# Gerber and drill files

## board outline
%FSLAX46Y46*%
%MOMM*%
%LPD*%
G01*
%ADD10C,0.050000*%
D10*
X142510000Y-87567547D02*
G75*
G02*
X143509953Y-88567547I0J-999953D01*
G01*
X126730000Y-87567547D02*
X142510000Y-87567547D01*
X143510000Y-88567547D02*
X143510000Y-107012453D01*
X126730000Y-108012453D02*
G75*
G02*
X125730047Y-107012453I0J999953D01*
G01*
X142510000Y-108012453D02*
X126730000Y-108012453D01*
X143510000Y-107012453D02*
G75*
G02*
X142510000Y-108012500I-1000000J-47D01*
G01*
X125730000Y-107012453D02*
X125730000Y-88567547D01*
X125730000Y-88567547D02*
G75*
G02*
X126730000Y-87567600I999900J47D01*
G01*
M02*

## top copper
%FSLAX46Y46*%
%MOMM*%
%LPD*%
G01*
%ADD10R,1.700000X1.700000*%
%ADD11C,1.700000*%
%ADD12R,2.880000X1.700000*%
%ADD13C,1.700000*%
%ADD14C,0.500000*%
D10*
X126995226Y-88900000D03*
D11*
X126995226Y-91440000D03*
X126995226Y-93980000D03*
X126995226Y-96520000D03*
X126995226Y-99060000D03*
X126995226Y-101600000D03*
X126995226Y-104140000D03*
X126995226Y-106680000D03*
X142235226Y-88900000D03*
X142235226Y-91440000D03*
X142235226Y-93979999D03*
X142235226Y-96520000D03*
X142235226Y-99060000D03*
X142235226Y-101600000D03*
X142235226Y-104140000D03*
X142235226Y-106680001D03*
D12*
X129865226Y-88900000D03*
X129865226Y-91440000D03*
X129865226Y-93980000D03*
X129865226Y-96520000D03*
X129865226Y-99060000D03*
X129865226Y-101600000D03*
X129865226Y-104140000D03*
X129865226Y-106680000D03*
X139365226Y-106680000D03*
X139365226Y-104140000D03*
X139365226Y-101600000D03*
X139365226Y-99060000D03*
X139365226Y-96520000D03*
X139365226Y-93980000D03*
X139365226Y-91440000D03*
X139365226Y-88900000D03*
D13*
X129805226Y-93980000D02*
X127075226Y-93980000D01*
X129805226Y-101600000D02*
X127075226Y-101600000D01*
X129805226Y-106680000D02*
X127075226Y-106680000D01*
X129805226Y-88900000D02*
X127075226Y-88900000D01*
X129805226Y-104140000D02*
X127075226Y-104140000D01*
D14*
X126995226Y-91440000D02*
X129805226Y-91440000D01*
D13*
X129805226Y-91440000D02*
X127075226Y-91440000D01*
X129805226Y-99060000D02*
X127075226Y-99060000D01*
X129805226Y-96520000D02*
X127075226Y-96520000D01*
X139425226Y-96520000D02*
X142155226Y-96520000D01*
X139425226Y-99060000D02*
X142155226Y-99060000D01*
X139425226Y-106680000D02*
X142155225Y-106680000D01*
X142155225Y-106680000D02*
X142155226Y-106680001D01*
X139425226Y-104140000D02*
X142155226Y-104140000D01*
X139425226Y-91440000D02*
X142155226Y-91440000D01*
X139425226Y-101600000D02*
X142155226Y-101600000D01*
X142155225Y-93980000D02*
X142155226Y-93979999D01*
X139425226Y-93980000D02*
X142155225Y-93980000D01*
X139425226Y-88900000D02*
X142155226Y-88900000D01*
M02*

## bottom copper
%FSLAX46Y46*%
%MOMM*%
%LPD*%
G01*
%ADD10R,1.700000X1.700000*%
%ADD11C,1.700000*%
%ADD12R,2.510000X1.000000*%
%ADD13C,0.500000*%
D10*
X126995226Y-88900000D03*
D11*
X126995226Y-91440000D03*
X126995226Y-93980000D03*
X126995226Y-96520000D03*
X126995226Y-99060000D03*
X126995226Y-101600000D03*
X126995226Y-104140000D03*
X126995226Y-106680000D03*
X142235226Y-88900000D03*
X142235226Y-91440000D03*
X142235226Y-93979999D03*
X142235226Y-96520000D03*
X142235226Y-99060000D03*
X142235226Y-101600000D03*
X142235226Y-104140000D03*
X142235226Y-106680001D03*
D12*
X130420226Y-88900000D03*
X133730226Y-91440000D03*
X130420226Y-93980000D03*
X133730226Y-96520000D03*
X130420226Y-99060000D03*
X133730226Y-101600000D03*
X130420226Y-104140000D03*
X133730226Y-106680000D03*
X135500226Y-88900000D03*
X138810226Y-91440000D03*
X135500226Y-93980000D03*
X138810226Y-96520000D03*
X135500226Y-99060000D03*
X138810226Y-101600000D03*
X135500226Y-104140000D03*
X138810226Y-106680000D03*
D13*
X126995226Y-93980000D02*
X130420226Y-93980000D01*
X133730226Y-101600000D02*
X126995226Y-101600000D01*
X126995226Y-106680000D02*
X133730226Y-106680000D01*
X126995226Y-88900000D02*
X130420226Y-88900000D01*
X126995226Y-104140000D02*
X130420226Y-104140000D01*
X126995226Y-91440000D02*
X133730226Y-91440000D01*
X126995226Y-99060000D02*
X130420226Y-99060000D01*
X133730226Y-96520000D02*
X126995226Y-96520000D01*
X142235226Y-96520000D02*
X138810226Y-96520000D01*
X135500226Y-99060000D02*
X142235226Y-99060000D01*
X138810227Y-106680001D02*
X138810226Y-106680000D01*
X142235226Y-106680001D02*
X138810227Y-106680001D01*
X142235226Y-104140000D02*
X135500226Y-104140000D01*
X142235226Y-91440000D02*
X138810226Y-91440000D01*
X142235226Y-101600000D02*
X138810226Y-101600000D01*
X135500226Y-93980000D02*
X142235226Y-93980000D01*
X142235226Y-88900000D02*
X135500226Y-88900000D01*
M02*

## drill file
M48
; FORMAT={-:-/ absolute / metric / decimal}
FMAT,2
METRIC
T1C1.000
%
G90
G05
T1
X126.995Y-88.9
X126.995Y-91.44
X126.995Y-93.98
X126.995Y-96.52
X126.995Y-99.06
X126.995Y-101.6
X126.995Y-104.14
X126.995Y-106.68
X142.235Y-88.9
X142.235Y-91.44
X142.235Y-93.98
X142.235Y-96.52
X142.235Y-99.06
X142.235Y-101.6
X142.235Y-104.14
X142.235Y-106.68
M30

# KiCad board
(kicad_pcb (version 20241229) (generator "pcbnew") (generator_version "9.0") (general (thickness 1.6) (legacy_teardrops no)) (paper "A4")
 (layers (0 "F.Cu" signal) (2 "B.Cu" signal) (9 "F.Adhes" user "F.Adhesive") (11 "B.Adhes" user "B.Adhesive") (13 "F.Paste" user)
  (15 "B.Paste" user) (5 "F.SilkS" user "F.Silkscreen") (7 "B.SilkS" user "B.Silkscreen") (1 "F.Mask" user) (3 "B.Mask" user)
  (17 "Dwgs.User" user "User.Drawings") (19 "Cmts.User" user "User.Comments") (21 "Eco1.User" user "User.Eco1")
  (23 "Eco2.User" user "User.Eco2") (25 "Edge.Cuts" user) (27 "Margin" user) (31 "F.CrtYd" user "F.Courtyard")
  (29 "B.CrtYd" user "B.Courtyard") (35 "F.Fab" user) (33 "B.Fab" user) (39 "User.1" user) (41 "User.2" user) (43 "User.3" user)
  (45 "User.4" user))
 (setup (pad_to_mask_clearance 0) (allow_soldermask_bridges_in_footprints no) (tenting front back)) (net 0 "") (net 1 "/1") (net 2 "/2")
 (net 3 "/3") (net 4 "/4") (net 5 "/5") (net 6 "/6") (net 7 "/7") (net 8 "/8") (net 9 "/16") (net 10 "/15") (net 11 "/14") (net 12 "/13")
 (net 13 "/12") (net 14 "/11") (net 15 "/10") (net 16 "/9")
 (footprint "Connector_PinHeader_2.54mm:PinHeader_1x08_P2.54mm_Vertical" (layer "F.Cu") (at 126.995226 88.9)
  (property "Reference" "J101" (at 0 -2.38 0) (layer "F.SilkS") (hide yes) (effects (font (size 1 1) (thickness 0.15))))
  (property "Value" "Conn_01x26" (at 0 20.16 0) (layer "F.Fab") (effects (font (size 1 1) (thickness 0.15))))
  (pad "1" thru_hole rect (at 0 0) (size 1.7 1.7) (drill 1) (layers "*.Cu" "*.Mask") (remove_unused_layers no) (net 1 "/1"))
  (pad "2" thru_hole circle (at 0 2.54) (size 1.7 1.7) (drill 1) (layers "*.Cu" "*.Mask") (remove_unused_layers no) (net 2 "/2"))
  (pad "3" thru_hole circle (at 0 5.08) (size 1.7 1.7) (drill 1) (layers "*.Cu" "*.Mask") (remove_unused_layers no) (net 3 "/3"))
  (pad "4" thru_hole circle (at 0 7.62) (size 1.7 1.7) (drill 1) (layers "*.Cu" "*.Mask") (remove_unused_layers no) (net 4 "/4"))
  (pad "5" thru_hole circle (at 0 10.16) (size 1.7 1.7) (drill 1) (layers "*.Cu" "*.Mask") (remove_unused_layers no) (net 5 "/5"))
  (pad "6" thru_hole circle (at 0 12.7) (size 1.7 1.7) (drill 1) (layers "*.Cu" "*.Mask") (remove_unused_layers no) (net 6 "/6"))
  (pad "7" thru_hole circle (at 0 15.24) (size 1.7 1.7) (drill 1) (layers "*.Cu" "*.Mask") (remove_unused_layers no) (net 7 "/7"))
  (pad "8" thru_hole circle (at 0 17.78) (size 1.7 1.7) (drill 1) (layers "*.Cu" "*.Mask") (remove_unused_layers no) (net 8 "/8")))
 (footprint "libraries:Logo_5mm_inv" (layer "F.Cu") (at 134.617351 90.17)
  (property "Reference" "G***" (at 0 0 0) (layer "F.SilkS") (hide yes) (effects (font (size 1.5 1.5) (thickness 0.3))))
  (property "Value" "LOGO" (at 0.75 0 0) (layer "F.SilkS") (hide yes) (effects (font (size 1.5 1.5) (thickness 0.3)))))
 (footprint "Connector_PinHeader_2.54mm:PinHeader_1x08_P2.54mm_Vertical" (layer "F.Cu") (at 142.235226 88.9)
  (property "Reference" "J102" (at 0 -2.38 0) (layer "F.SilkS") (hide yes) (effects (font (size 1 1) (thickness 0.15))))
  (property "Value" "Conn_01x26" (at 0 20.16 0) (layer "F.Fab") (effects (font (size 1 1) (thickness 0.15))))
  (pad "1" thru_hole circle (at 0 0) (size 1.7 1.7) (drill 1) (layers "*.Cu" "*.Mask") (remove_unused_layers no) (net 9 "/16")
   (thermal_bridge_angle 90))
  (pad "2" thru_hole circle (at 0 2.54) (size 1.7 1.7) (drill 1) (layers "*.Cu" "*.Mask") (remove_unused_layers no) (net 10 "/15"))
  (pad "3" thru_hole circle (at 0 5.079999) (size 1.7 1.7) (drill 1) (layers "*.Cu" "*.Mask") (remove_unused_layers no) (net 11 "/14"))
  (pad "4" thru_hole circle (at 0 7.62) (size 1.7 1.7) (drill 1) (layers "*.Cu" "*.Mask") (remove_unused_layers no) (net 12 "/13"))
  (pad "5" thru_hole circle (at 0 10.16) (size 1.7 1.7) (drill 1) (layers "*.Cu" "*.Mask") (remove_unused_layers no) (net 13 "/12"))
  (pad "6" thru_hole circle (at 0 12.7) (size 1.7 1.7) (drill 1) (layers "*.Cu" "*.Mask") (remove_unused_layers no) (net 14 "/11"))
  (pad "7" thru_hole circle (at 0 15.24) (size 1.7 1.7) (drill 1) (layers "*.Cu" "*.Mask") (remove_unused_layers no) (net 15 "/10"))
  (pad "8" thru_hole circle (at 0 17.780001) (size 1.7 1.7) (drill 1) (layers "*.Cu" "*.Mask") (remove_unused_layers no) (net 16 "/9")))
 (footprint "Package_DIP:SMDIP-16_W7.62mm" (layer "F.Cu") (at 134.615226 97.79)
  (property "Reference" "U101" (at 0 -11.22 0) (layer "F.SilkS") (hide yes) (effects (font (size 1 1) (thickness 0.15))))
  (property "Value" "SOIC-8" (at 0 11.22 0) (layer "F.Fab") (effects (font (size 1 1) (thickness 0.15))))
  (pad "1" smd rect (at -4.75 -8.89) (size 2.88 1.7) (layers "F.Cu" "F.Mask" "F.Paste") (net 1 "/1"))
  (pad "2" smd rect (at -4.75 -6.35) (size 2.88 1.7) (layers "F.Cu" "F.Mask" "F.Paste") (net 2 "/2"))
  (pad "3" smd rect (at -4.75 -3.81) (size 2.88 1.7) (layers "F.Cu" "F.Mask" "F.Paste") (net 3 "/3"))
  (pad "4" smd rect (at -4.75 -1.27) (size 2.88 1.7) (layers "F.Cu" "F.Mask" "F.Paste") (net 4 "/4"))
  (pad "5" smd rect (at -4.75 1.27) (size 2.88 1.7) (layers "F.Cu" "F.Mask" "F.Paste") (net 5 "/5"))
  (pad "6" smd rect (at -4.75 3.81) (size 2.88 1.7) (layers "F.Cu" "F.Mask" "F.Paste") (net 6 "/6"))
  (pad "7" smd rect (at -4.75 6.35) (size 2.88 1.7) (layers "F.Cu" "F.Mask" "F.Paste") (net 7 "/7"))
  (pad "8" smd rect (at -4.75 8.89) (size 2.88 1.7) (layers "F.Cu" "F.Mask" "F.Paste") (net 8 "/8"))
  (pad "9" smd rect (at 4.75 8.89) (size 2.88 1.7) (layers "F.Cu" "F.Mask" "F.Paste") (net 16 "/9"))
  (pad "10" smd rect (at 4.75 6.35) (size 2.88 1.7) (layers "F.Cu" "F.Mask" "F.Paste") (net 15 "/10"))
  (pad "11" smd rect (at 4.75 3.81) (size 2.88 1.7) (layers "F.Cu" "F.Mask" "F.Paste") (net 14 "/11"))
  (pad "12" smd rect (at 4.75 1.27) (size 2.88 1.7) (layers "F.Cu" "F.Mask" "F.Paste") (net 13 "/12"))
  (pad "13" smd rect (at 4.75 -1.27) (size 2.88 1.7) (layers "F.Cu" "F.Mask" "F.Paste") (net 12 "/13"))
  (pad "14" smd rect (at 4.75 -3.81) (size 2.88 1.7) (layers "F.Cu" "F.Mask" "F.Paste") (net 11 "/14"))
  (pad "15" smd rect (at 4.75 -6.35) (size 2.88 1.7) (layers "F.Cu" "F.Mask" "F.Paste") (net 10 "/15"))
  (pad "16" smd rect (at 4.75 -8.89) (size 2.88 1.7) (layers "F.Cu" "F.Mask" "F.Paste") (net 9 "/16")))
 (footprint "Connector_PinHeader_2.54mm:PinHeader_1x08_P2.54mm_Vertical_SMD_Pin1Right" (layer "B.Cu") (at 132.075226 97.79 180)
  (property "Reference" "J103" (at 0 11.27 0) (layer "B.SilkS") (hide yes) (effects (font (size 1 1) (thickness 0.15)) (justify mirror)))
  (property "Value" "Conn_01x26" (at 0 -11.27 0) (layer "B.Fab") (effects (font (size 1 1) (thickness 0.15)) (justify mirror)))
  (pad "1" smd rect (at 1.655 8.89 180) (size 2.51 1) (layers "B.Cu" "B.Mask" "B.Paste") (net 1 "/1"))
  (pad "2" smd rect (at -1.655 6.35 180) (size 2.51 1) (layers "B.Cu" "B.Mask" "B.Paste") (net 2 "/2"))
  (pad "3" smd rect (at 1.655 3.81 180) (size 2.51 1) (layers "B.Cu" "B.Mask" "B.Paste") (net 3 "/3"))
  (pad "4" smd rect (at -1.655 1.27 180) (size 2.51 1) (layers "B.Cu" "B.Mask" "B.Paste") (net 4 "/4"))
  (pad "5" smd rect (at 1.655 -1.27 180) (size 2.51 1) (layers "B.Cu" "B.Mask" "B.Paste") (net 5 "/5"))
  (pad "6" smd rect (at -1.655 -3.81 180) (size 2.51 1) (layers "B.Cu" "B.Mask" "B.Paste") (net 6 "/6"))
  (pad "7" smd rect (at 1.655 -6.35 180) (size 2.51 1) (layers "B.Cu" "B.Mask" "B.Paste") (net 7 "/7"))
  (pad "8" smd rect (at -1.655 -8.89 180) (size 2.51 1) (layers "B.Cu" "B.Mask" "B.Paste") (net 8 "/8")))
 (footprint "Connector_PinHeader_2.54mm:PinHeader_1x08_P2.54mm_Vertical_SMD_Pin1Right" (layer "B.Cu") (at 137.155226 97.79 180)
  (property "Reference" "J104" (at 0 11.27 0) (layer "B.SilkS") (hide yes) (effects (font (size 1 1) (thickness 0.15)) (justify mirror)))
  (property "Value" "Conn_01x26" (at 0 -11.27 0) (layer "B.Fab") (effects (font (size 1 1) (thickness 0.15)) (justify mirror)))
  (pad "1" smd rect (at 1.655 8.89 180) (size 2.51 1) (layers "B.Cu" "B.Mask" "B.Paste") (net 9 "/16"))
  (pad "2" smd rect (at -1.655 6.35 180) (size 2.51 1) (layers "B.Cu" "B.Mask" "B.Paste") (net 10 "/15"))
  (pad "3" smd rect (at 1.655 3.81 180) (size 2.51 1) (layers "B.Cu" "B.Mask" "B.Paste") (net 11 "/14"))
  (pad "4" smd rect (at -1.655 1.27 180) (size 2.51 1) (layers "B.Cu" "B.Mask" "B.Paste") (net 12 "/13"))
  (pad "5" smd rect (at 1.655 -1.27 180) (size 2.51 1) (layers "B.Cu" "B.Mask" "B.Paste") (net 13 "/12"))
  (pad "6" smd rect (at -1.655 -3.81 180) (size 2.51 1) (layers "B.Cu" "B.Mask" "B.Paste") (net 14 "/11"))
  (pad "7" smd rect (at 1.655 -6.35 180) (size 2.51 1) (layers "B.Cu" "B.Mask" "B.Paste") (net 15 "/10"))
  (pad "8" smd rect (at -1.655 -8.89 180) (size 2.51 1) (layers "B.Cu" "B.Mask" "B.Paste") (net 16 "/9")))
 (gr_arc (start 142.51 87.567547) (mid 143.217107 87.86044) (end 143.51 88.567547) (stroke (width 0.05) (type default)) (layer "Edge.Cuts"))
 (gr_line (start 126.73 87.567547) (end 142.51 87.567547) (stroke (width 0.05) (type default)) (layer "Edge.Cuts"))
 (gr_line (start 143.51 88.567547) (end 143.51 107.012453) (stroke (width 0.05) (type default)) (layer "Edge.Cuts"))
 (gr_arc (start 126.73 108.012453) (mid 126.022893 107.71956) (end 125.73 107.012453) (stroke (width 0.05) (type default))
  (layer "Edge.Cuts"))
 (gr_line (start 142.51 108.012453) (end 126.73 108.012453) (stroke (width 0.05) (type default)) (layer "Edge.Cuts"))
 (gr_arc (start 143.51 107.012453) (mid 143.217107 107.71956) (end 142.51 108.012453) (stroke (width 0.05) (type default))
  (layer "Edge.Cuts"))
 (gr_line (start 125.73 107.012453) (end 125.73 88.567547) (stroke (width 0.05) (type default)) (layer "Edge.Cuts"))
 (gr_arc (start 125.73 88.567547) (mid 126.022877 87.86041) (end 126.73 87.567547) (stroke (width 0.05) (type default)) (layer "Edge.Cuts"))
 (segment (start 129.805226 93.98) (end 127.075226 93.98) (width 1.7) (layer "F.Cu") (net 3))
 (segment (start 126.995226 93.98) (end 130.420226 93.98) (width 0.5) (layer "B.Cu") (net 3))
 (segment (start 129.805226 101.6) (end 127.075226 101.6) (width 1.7) (layer "F.Cu") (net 6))
 (segment (start 133.730226 101.6) (end 126.995226 101.6) (width 0.5) (layer "B.Cu") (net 6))
 (segment (start 129.805226 106.68) (end 127.075226 106.68) (width 1.7) (layer "F.Cu") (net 8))
 (segment (start 126.995226 106.68) (end 133.730226 106.68) (width 0.5) (layer "B.Cu") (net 8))
 (segment (start 129.805226 88.9) (end 127.075226 88.9) (width 1.7) (layer "F.Cu") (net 1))
 (segment (start 126.995226 88.9) (end 130.420226 88.9) (width 0.5) (layer "B.Cu") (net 1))
 (segment (start 129.805226 104.14) (end 127.075226 104.14) (width 1.7) (layer "F.Cu") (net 7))
 (segment (start 126.995226 104.14) (end 130.420226 104.14) (width 0.5) (layer "B.Cu") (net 7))
 (segment (start 126.995226 91.44) (end 129.805226 91.44) (width 0.5) (layer "F.Cu") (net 2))
 (segment (start 129.805226 91.44) (end 127.075226 91.44) (width 1.7) (layer "F.Cu") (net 2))
 (segment (start 126.995226 91.44) (end 133.730226 91.44) (width 0.5) (layer "B.Cu") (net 2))
 (segment (start 129.805226 99.06) (end 127.075226 99.06) (width 1.7) (layer "F.Cu") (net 5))
 (segment (start 126.995226 99.06) (end 130.420226 99.06) (width 0.5) (layer "B.Cu") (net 5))
 (segment (start 129.805226 96.52) (end 127.075226 96.52) (width 1.7) (layer "F.Cu") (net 4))
 (segment (start 133.730226 96.52) (end 126.995226 96.52) (width 0.5) (layer "B.Cu") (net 4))
 (segment (start 139.425226 96.52) (end 142.155226 96.52) (width 1.7) (layer "F.Cu") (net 12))
 (segment (start 142.235226 96.52) (end 138.810226 96.52) (width 0.5) (layer "B.Cu") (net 12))
 (segment (start 139.425226 99.06) (end 142.155226 99.06) (width 1.7) (layer "F.Cu") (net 13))
 (segment (start 135.500226 99.06) (end 142.235226 99.06) (width 0.5) (layer "B.Cu") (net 13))
 (segment (start 139.425226 106.68) (end 142.155225 106.68) (width 1.7) (layer "F.Cu") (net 16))
 (segment (start 142.155225 106.68) (end 142.155226 106.680001) (width 1.7) (layer "F.Cu") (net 16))
 (segment (start 138.810227 106.680001) (end 138.810226 106.68) (width 0.5) (layer "B.Cu") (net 16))
 (segment (start 142.235226 106.680001) (end 138.810227 106.680001) (width 0.5) (layer "B.Cu") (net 16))
 (segment (start 139.425226 104.14) (end 142.155226 104.14) (width 1.7) (layer "F.Cu") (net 15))
 (segment (start 142.235226 104.14) (end 135.500226 104.14) (width 0.5) (layer "B.Cu") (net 15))
 (segment (start 139.425226 91.44) (end 142.155226 91.44) (width 1.7) (layer "F.Cu") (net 10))
 (segment (start 142.235226 91.44) (end 138.810226 91.44) (width 0.5) (layer "B.Cu") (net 10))
 (segment (start 139.425226 101.6) (end 142.155226 101.6) (width 1.7) (layer "F.Cu") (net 14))
 (segment (start 142.235226 101.6) (end 138.810226 101.6) (width 0.5) (layer "B.Cu") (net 14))
 (segment (start 142.155225 93.98) (end 142.155226 93.979999) (width 1.7) (layer "F.Cu") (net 11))
 (segment (start 139.425226 93.98) (end 142.155225 93.98) (width 1.7) (layer "F.Cu") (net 11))
 (segment (start 135.500226 93.98) (end 142.235226 93.98) (width 0.5) (layer "B.Cu") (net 11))
 (segment (start 139.425226 88.9) (end 142.155226 88.9) (width 1.7) (layer "F.Cu") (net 9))
 (segment (start 142.235226 88.9) (end 135.500226 88.9) (width 0.5) (layer "B.Cu") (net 9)))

